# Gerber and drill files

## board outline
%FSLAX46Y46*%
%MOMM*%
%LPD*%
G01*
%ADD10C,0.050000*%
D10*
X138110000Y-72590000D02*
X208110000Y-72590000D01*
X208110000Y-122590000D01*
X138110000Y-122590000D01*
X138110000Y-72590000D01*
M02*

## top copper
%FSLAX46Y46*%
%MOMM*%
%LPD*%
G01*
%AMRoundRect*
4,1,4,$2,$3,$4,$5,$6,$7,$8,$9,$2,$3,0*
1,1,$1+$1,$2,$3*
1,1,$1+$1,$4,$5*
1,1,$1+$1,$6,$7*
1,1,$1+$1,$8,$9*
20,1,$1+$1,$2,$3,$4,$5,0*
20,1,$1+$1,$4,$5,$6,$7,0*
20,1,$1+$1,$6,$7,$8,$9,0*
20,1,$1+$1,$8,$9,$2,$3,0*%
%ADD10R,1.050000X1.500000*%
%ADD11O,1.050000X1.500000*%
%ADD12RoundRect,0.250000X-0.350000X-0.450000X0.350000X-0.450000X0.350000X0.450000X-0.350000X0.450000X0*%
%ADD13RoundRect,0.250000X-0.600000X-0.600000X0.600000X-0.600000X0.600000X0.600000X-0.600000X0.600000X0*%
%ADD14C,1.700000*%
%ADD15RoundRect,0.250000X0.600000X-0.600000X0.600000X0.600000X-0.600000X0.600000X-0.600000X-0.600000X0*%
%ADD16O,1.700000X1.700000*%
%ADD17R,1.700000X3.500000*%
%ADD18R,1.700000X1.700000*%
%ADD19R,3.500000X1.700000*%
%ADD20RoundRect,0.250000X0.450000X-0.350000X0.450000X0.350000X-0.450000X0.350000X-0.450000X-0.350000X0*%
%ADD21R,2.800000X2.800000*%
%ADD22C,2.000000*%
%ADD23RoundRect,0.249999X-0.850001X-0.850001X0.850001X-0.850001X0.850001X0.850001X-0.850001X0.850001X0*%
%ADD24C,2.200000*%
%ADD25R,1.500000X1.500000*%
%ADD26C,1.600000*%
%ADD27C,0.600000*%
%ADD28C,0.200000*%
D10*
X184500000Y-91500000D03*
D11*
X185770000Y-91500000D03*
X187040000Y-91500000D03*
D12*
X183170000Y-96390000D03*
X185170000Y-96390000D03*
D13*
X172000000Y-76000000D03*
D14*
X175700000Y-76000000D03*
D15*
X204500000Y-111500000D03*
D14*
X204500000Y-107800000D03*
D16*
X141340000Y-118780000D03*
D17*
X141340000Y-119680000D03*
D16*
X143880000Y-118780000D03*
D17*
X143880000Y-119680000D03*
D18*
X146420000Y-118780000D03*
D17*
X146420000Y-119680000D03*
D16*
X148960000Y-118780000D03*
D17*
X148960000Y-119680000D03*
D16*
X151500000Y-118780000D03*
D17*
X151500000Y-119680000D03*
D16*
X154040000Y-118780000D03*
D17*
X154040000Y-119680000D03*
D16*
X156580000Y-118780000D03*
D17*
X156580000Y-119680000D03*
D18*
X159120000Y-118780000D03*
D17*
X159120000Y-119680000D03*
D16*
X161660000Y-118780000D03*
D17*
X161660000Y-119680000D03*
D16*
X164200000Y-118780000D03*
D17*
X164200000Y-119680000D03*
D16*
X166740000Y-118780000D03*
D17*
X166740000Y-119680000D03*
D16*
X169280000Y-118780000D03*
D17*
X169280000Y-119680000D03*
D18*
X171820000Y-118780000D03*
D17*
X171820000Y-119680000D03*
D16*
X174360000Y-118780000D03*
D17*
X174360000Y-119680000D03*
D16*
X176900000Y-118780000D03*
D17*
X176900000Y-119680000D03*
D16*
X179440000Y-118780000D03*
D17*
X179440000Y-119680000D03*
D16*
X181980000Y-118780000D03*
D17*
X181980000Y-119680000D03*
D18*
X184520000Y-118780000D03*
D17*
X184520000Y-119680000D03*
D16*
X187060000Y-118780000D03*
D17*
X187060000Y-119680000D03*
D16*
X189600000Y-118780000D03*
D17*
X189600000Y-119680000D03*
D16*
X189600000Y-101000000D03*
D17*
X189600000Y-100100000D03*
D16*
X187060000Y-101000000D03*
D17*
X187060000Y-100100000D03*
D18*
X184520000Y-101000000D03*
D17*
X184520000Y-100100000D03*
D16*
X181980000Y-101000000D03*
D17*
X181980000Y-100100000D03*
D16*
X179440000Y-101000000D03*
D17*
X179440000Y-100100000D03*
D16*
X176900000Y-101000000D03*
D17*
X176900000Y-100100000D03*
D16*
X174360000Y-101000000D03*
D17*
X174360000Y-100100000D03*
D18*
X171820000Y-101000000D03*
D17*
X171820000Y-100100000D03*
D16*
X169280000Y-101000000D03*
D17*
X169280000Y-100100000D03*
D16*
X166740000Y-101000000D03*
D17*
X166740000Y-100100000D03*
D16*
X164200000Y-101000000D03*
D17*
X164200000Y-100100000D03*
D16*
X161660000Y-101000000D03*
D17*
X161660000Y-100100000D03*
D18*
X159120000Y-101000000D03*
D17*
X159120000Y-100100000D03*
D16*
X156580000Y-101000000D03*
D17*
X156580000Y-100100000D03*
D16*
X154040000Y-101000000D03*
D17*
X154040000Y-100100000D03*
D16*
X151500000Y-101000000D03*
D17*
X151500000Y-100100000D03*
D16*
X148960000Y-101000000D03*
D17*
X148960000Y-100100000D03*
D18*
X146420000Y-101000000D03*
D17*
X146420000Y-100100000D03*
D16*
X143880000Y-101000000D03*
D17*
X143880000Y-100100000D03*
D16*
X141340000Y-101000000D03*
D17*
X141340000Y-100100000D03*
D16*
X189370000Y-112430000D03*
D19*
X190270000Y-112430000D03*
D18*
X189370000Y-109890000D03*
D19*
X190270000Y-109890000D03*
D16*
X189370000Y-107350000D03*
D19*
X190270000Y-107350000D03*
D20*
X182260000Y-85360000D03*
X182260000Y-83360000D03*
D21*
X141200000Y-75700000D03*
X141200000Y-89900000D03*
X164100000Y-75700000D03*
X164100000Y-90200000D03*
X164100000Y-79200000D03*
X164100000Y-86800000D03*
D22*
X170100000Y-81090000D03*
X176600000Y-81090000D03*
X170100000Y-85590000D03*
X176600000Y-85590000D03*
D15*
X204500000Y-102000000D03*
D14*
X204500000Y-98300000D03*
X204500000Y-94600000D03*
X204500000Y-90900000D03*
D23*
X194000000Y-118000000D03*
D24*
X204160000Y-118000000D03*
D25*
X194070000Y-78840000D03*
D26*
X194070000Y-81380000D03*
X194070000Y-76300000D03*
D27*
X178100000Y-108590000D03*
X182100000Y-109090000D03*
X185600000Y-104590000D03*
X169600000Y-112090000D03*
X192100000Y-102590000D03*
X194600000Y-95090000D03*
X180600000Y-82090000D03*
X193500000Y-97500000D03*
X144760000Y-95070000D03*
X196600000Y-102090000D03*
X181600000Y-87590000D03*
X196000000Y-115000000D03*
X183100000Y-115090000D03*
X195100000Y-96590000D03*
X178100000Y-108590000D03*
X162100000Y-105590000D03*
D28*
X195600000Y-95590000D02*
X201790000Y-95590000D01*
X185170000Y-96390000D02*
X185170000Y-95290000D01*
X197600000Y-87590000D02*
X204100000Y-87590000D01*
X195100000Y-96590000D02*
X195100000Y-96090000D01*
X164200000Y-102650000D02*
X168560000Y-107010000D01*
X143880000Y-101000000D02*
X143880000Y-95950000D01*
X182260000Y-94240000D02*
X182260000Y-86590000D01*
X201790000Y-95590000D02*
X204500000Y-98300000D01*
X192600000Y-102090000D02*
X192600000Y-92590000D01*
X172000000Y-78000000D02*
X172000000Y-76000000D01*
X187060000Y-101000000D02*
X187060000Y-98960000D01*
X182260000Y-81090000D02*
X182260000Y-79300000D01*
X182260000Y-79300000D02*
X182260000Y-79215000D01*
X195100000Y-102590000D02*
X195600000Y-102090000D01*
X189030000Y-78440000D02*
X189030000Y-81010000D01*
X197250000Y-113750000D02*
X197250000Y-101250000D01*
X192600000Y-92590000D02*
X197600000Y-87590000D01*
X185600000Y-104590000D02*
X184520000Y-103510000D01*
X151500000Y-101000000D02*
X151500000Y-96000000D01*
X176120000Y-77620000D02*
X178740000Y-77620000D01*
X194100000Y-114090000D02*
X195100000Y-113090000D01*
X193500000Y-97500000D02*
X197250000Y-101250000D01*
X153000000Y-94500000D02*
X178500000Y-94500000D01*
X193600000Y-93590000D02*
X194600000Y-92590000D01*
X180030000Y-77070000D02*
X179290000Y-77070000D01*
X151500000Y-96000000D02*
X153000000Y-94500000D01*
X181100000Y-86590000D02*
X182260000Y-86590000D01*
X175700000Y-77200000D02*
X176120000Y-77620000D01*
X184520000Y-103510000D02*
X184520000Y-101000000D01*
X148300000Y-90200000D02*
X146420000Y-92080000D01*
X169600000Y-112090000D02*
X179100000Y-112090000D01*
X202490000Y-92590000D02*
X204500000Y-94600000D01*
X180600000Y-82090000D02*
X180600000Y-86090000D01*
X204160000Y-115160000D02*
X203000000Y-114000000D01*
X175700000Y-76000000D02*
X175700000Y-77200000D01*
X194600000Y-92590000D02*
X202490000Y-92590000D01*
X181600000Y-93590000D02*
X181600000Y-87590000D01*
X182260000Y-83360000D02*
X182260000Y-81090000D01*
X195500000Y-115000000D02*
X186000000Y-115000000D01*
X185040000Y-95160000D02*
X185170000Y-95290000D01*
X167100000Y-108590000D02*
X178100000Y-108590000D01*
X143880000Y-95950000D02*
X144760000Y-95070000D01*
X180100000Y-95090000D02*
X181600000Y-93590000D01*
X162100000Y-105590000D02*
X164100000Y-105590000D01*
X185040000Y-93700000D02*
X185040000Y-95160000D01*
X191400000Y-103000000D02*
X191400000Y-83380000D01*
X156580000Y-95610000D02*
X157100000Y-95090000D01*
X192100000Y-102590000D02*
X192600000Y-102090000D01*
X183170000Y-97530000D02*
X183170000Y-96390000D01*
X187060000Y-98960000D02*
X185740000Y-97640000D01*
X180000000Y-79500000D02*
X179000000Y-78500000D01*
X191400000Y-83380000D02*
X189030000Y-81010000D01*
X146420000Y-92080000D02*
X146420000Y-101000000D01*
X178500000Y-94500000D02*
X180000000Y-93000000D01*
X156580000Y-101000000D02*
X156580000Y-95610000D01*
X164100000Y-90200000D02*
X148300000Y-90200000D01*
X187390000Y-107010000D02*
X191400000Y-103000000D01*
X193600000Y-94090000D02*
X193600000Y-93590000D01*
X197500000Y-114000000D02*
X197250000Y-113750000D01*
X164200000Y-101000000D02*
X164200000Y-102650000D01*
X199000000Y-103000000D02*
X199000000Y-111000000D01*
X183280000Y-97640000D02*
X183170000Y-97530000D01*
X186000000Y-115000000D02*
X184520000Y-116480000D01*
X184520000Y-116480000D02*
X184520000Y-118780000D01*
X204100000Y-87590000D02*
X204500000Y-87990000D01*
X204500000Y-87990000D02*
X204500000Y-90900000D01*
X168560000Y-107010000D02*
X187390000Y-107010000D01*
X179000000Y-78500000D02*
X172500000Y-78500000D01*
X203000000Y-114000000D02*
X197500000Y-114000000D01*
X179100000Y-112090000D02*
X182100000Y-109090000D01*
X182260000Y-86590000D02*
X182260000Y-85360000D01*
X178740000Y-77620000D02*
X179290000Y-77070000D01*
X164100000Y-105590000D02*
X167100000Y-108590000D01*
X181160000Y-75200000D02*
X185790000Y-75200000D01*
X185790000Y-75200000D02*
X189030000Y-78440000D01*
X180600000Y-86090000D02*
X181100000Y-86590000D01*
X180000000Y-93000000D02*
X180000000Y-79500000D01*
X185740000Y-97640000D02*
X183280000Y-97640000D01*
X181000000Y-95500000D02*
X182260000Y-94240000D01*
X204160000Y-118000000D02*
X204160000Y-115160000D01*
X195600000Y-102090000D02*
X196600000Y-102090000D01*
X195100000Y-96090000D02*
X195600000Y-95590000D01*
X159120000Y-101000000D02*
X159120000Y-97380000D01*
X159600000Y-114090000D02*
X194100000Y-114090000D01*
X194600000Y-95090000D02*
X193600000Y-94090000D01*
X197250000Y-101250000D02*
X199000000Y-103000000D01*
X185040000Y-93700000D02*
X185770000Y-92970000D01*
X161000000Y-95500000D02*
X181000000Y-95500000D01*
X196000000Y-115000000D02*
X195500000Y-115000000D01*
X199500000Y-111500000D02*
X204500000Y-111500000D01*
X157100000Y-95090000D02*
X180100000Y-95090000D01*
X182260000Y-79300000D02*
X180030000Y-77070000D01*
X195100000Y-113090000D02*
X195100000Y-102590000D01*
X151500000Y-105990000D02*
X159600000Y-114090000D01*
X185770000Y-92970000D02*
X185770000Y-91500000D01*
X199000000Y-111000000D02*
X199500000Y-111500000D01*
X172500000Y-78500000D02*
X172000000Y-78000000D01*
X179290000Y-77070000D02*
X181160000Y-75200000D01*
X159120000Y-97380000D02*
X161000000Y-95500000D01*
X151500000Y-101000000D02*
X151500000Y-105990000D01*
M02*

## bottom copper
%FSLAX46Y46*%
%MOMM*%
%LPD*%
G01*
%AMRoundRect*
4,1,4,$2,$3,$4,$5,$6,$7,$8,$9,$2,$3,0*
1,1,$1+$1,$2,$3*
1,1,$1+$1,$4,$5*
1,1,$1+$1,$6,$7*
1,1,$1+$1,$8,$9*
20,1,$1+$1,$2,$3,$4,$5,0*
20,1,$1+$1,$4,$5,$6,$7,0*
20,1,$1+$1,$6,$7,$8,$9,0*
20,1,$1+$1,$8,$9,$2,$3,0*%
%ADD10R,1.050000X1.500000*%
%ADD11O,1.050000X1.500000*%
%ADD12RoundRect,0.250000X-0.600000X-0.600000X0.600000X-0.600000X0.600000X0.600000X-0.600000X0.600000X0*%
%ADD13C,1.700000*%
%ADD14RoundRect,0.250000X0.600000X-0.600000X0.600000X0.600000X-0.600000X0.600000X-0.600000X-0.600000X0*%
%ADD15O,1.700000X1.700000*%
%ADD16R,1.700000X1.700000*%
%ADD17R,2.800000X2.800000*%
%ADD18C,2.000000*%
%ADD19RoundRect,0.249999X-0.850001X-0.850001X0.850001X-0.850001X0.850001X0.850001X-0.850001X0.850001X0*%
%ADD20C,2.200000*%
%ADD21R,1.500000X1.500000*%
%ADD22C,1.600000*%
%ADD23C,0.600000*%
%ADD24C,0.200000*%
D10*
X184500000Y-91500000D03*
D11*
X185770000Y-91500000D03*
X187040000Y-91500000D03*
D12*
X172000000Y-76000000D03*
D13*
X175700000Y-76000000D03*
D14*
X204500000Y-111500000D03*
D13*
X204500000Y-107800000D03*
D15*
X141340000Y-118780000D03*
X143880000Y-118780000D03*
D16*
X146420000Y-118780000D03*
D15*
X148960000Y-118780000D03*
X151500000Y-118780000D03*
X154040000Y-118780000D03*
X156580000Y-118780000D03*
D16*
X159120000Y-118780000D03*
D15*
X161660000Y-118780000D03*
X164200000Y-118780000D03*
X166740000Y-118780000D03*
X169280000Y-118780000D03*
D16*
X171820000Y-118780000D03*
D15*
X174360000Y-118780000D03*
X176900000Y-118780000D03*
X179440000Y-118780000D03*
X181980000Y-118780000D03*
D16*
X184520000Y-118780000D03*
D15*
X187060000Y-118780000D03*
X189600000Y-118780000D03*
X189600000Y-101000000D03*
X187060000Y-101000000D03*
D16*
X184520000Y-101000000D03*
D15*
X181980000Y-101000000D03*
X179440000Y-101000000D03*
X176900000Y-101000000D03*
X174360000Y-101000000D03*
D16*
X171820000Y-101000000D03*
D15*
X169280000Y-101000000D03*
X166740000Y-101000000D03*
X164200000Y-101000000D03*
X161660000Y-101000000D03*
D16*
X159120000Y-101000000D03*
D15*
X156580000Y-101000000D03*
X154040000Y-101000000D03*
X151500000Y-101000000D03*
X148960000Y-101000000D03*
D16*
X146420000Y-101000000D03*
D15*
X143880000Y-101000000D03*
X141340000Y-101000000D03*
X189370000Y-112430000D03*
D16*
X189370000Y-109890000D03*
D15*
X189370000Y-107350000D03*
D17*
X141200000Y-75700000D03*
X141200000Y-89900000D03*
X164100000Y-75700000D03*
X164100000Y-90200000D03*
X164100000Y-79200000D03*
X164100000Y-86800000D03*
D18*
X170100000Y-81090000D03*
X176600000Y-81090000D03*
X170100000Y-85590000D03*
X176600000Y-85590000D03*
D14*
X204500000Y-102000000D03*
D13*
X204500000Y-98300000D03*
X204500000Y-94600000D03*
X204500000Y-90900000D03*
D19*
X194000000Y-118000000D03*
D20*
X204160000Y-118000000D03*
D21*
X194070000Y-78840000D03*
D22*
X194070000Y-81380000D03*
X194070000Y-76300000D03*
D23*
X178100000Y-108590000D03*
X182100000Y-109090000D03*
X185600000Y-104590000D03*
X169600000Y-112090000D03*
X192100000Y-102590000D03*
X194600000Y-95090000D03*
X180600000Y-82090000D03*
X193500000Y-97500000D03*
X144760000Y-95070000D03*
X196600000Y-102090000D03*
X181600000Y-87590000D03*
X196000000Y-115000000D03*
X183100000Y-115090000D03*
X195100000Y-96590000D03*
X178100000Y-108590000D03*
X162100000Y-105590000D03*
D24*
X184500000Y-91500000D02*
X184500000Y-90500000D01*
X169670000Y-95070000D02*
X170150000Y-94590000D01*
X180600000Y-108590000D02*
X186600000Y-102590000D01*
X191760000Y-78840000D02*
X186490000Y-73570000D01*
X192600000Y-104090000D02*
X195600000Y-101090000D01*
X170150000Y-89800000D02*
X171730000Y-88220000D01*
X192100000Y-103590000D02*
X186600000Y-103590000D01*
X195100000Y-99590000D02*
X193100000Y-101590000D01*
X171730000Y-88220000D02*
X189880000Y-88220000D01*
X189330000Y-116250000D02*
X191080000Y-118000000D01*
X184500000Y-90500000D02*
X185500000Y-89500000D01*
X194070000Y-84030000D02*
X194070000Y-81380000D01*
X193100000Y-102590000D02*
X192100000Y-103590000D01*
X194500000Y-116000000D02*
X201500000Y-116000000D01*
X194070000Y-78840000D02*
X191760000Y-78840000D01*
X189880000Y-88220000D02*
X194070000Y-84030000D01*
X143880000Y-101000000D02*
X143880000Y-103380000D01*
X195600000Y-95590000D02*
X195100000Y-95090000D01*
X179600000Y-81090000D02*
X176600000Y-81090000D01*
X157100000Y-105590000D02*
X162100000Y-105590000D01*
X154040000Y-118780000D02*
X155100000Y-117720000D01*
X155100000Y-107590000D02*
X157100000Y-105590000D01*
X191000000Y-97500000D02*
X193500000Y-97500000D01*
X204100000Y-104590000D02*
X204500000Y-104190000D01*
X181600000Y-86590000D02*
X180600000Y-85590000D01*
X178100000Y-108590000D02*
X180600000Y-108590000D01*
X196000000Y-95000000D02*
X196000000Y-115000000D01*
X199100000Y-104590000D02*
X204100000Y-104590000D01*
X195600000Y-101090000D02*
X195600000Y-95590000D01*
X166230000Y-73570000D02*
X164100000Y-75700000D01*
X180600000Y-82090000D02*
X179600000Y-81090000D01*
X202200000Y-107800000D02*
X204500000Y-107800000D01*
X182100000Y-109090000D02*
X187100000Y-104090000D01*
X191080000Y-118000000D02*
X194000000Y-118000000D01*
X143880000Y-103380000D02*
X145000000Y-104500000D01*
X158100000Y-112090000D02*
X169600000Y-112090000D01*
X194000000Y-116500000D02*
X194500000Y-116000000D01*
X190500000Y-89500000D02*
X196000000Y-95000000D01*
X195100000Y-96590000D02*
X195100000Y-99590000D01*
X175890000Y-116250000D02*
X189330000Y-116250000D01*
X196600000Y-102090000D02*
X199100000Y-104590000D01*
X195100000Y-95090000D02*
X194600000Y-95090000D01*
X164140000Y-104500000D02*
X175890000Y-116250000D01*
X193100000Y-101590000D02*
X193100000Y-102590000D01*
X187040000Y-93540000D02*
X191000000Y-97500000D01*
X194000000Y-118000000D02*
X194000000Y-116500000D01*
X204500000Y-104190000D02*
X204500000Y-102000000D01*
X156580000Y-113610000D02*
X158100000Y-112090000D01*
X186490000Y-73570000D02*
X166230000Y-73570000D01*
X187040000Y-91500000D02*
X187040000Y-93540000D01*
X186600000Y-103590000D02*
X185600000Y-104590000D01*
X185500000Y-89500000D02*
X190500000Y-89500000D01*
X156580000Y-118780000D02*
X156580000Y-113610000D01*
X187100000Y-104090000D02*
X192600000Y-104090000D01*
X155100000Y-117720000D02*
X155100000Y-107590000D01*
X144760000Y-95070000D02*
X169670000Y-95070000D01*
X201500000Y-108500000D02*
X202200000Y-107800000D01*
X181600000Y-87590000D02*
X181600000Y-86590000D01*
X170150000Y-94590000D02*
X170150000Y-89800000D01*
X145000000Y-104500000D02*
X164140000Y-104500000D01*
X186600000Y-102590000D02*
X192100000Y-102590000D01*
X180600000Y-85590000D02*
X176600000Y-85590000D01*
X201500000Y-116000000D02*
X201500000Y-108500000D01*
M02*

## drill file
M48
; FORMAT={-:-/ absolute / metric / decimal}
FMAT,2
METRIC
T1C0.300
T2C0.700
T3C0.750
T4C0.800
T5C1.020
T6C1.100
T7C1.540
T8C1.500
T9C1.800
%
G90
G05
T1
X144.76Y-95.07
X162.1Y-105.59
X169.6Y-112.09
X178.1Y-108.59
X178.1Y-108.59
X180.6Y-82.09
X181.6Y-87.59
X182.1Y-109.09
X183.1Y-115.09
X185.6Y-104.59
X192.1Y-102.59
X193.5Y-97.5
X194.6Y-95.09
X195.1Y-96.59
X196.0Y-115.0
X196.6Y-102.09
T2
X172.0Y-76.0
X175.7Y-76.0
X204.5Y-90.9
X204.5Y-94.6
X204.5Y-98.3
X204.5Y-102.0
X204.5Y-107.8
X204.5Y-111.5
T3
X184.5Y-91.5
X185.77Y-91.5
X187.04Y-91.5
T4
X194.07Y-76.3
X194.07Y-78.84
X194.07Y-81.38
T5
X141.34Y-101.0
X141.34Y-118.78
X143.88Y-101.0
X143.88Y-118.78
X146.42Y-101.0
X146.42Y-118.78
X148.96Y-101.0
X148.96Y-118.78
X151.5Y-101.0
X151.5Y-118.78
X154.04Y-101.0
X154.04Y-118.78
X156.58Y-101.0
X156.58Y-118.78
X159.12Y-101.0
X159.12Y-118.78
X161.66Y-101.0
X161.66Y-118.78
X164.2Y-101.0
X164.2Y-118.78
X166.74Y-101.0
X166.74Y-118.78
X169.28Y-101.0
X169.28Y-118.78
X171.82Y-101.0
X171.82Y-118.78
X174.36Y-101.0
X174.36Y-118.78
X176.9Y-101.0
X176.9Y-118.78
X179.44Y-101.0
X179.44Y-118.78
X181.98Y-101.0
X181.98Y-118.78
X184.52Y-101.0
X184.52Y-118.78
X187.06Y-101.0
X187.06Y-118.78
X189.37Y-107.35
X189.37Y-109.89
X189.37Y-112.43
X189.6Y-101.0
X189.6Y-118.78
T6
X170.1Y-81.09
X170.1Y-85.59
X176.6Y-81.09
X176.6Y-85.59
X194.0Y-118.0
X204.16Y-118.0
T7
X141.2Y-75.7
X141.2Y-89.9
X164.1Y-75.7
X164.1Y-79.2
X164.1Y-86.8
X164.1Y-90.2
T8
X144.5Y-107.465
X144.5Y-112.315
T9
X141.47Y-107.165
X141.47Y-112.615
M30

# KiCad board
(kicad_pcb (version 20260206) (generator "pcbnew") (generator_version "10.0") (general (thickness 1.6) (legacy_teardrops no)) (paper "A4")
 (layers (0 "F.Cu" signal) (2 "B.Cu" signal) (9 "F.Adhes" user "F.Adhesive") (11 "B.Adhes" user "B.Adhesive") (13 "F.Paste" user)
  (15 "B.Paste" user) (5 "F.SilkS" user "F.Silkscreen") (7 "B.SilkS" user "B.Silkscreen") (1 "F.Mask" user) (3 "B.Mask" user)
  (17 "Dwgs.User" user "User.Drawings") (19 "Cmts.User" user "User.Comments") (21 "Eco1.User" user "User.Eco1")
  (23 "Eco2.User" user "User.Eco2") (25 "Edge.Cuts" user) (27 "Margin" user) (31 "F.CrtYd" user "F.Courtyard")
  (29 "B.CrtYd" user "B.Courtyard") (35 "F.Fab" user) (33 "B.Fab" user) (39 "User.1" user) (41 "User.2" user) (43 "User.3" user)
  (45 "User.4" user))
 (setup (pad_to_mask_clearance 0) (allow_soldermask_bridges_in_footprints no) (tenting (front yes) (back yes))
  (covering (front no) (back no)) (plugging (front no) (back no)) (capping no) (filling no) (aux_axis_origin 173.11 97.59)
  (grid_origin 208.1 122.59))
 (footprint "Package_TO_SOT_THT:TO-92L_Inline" (layer "F.Cu") (at 184.5 91.5)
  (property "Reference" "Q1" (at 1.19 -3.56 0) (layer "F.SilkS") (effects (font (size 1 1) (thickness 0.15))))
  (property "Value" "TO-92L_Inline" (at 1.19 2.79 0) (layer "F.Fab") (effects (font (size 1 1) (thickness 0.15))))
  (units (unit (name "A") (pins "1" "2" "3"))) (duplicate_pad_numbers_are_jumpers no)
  (pad "1" thru_hole rect (at 0 0) (size 1.05 1.5) (drill 0.75) (layers "*.Cu" "*.Mask") (remove_unused_layers no))
  (pad "2" thru_hole oval (at 1.27 0) (size 1.05 1.5) (drill 0.75) (layers "*.Cu" "*.Mask") (remove_unused_layers no))
  (pad "3" thru_hole oval (at 2.54 0) (size 1.05 1.5) (drill 0.75) (layers "*.Cu" "*.Mask") (remove_unused_layers no)))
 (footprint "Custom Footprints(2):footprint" (layer "F.Cu") (at 202 78.55)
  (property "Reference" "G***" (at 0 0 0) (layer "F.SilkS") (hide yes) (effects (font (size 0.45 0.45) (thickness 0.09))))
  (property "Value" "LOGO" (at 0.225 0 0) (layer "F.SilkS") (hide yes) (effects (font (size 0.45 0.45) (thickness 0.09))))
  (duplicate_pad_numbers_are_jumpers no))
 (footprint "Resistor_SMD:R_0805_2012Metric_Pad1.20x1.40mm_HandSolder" (layer "F.Cu") (at 184.17 96.39)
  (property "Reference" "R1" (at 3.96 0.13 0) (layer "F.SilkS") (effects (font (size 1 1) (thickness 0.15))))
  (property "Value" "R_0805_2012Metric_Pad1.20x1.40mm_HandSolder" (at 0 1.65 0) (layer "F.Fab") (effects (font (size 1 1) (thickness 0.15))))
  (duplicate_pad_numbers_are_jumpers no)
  (pad "1" smd roundrect (at -1 0) (size 1.2 1.4) (layers "F.Cu" "F.Mask" "F.Paste") (roundrect_rratio 0.208333))
  (pad "2" smd roundrect (at 1 0) (size 1.2 1.4) (layers "F.Cu" "F.Mask" "F.Paste") (roundrect_rratio 0.208333)))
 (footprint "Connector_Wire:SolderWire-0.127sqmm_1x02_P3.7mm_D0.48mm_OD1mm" (layer "F.Cu") (at 172 76)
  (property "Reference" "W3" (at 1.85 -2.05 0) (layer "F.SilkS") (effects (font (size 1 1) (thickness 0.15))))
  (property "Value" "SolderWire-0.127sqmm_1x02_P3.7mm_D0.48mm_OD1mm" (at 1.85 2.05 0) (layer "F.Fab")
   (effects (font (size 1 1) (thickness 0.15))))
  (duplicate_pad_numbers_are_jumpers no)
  (pad "1" thru_hole roundrect (at 0 0) (size 1.7 1.7) (drill 0.7) (layers "*.Cu" "*.Mask") (remove_unused_layers no)
   (roundrect_rratio 0.147059))
  (pad "2" thru_hole circle (at 3.7 0) (size 1.7 1.7) (drill 0.7) (layers "*.Cu" "*.Mask") (remove_unused_layers no)))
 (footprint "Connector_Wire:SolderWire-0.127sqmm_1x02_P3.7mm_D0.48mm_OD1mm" (layer "F.Cu") (at 204.5 111.5 90)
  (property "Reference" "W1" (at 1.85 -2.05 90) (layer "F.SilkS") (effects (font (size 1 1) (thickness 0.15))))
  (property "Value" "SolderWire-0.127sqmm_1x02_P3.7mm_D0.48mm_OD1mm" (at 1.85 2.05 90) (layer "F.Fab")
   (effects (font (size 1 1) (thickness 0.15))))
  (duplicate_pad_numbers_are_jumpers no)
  (pad "1" thru_hole roundrect (at 0 0 90) (size 1.7 1.7) (drill 0.7) (layers "*.Cu" "*.Mask") (remove_unused_layers no)
   (roundrect_rratio 0.147059))
  (pad "2" thru_hole circle (at 3.7 0 90) (size 1.7 1.7) (drill 0.7) (layers "*.Cu" "*.Mask") (remove_unused_layers no)))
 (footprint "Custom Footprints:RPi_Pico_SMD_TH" (layer "F.Cu") (at 165.47 109.89 90)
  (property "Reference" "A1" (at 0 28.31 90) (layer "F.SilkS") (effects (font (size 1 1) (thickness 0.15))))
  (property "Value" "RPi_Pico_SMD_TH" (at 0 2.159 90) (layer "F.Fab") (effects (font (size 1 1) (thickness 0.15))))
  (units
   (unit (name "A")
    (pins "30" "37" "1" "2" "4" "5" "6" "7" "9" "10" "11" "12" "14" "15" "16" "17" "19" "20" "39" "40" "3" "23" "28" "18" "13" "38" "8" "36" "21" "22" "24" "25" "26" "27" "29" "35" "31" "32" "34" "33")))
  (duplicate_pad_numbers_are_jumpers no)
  (pad "" np_thru_hole oval (at -2.725 -24 90) (size 1.8 1.8) (drill 1.8) (layers "*.Cu" "*.Mask"))
  (pad "" np_thru_hole oval (at -2.425 -20.97 90) (size 1.5 1.5) (drill 1.5) (layers "*.Cu" "*.Mask"))
  (pad "" np_thru_hole oval (at 2.425 -20.97 90) (size 1.5 1.5) (drill 1.5) (layers "*.Cu" "*.Mask"))
  (pad "" np_thru_hole oval (at 2.725 -24 90) (size 1.8 1.8) (drill 1.8) (layers "*.Cu" "*.Mask"))
  (pad "1" thru_hole oval (at -8.89 -24.13 90) (size 1.7 1.7) (drill 1.02) (layers "*.Cu" "*.Mask") (remove_unused_layers no))
  (pad "1" smd rect (at -8.89 -24.13 90) (size 3.5 1.7) (drill (offset -0.9 0)) (layers "F.Cu" "F.Mask"))
  (pad "2" thru_hole oval (at -8.89 -21.59 90) (size 1.7 1.7) (drill 1.02) (layers "*.Cu" "*.Mask") (remove_unused_layers no))
  (pad "2" smd rect (at -8.89 -21.59 90) (size 3.5 1.7) (drill (offset -0.9 0)) (layers "F.Cu" "F.Mask"))
  (pad "3" thru_hole rect (at -8.89 -19.05 90) (size 1.7 1.7) (drill 1.02) (layers "*.Cu" "*.Mask") (remove_unused_layers no))
  (pad "3" smd rect (at -8.89 -19.05 90) (size 3.5 1.7) (drill (offset -0.9 0)) (layers "F.Cu" "F.Mask"))
  (pad "4" thru_hole oval (at -8.89 -16.51 90) (size 1.7 1.7) (drill 1.02) (layers "*.Cu" "*.Mask") (remove_unused_layers no))
  (pad "4" smd rect (at -8.89 -16.51 90) (size 3.5 1.7) (drill (offset -0.9 0)) (layers "F.Cu" "F.Mask"))
  (pad "5" thru_hole oval (at -8.89 -13.97 90) (size 1.7 1.7) (drill 1.02) (layers "*.Cu" "*.Mask") (remove_unused_layers no))
  (pad "5" smd rect (at -8.89 -13.97 90) (size 3.5 1.7) (drill (offset -0.9 0)) (layers "F.Cu" "F.Mask"))
  (pad "6" thru_hole oval (at -8.89 -11.43 90) (size 1.7 1.7) (drill 1.02) (layers "*.Cu" "*.Mask") (remove_unused_layers no))
  (pad "6" smd rect (at -8.89 -11.43 90) (size 3.5 1.7) (drill (offset -0.9 0)) (layers "F.Cu" "F.Mask"))
  (pad "7" thru_hole oval (at -8.89 -8.89 90) (size 1.7 1.7) (drill 1.02) (layers "*.Cu" "*.Mask") (remove_unused_layers no))
  (pad "7" smd rect (at -8.89 -8.89 90) (size 3.5 1.7) (drill (offset -0.9 0)) (layers "F.Cu" "F.Mask"))
  (pad "8" thru_hole rect (at -8.89 -6.35 90) (size 1.7 1.7) (drill 1.02) (layers "*.Cu" "*.Mask") (remove_unused_layers no))
  (pad "8" smd rect (at -8.89 -6.35 90) (size 3.5 1.7) (drill (offset -0.9 0)) (layers "F.Cu" "F.Mask"))
  (pad "9" thru_hole oval (at -8.89 -3.81 90) (size 1.7 1.7) (drill 1.02) (layers "*.Cu" "*.Mask") (remove_unused_layers no))
  (pad "9" smd rect (at -8.89 -3.81 90) (size 3.5 1.7) (drill (offset -0.9 0)) (layers "F.Cu" "F.Mask"))
  (pad "10" thru_hole oval (at -8.89 -1.27 90) (size 1.7 1.7) (drill 1.02) (layers "*.Cu" "*.Mask") (remove_unused_layers no))
  (pad "10" smd rect (at -8.89 -1.27 90) (size 3.5 1.7) (drill (offset -0.9 0)) (layers "F.Cu" "F.Mask"))
  (pad "11" thru_hole oval (at -8.89 1.27 90) (size 1.7 1.7) (drill 1.02) (layers "*.Cu" "*.Mask") (remove_unused_layers no))
  (pad "11" smd rect (at -8.89 1.27 90) (size 3.5 1.7) (drill (offset -0.9 0)) (layers "F.Cu" "F.Mask"))
  (pad "12" thru_hole oval (at -8.89 3.81 90) (size 1.7 1.7) (drill 1.02) (layers "*.Cu" "*.Mask") (remove_unused_layers no))
  (pad "12" smd rect (at -8.89 3.81 90) (size 3.5 1.7) (drill (offset -0.9 0)) (layers "F.Cu" "F.Mask"))
  (pad "13" thru_hole rect (at -8.89 6.35 90) (size 1.7 1.7) (drill 1.02) (layers "*.Cu" "*.Mask") (remove_unused_layers no))
  (pad "13" smd rect (at -8.89 6.35 90) (size 3.5 1.7) (drill (offset -0.9 0)) (layers "F.Cu" "F.Mask"))
  (pad "14" thru_hole oval (at -8.89 8.89 90) (size 1.7 1.7) (drill 1.02) (layers "*.Cu" "*.Mask") (remove_unused_layers no))
  (pad "14" smd rect (at -8.89 8.89 90) (size 3.5 1.7) (drill (offset -0.9 0)) (layers "F.Cu" "F.Mask"))
  (pad "15" thru_hole oval (at -8.89 11.43 90) (size 1.7 1.7) (drill 1.02) (layers "*.Cu" "*.Mask") (remove_unused_layers no))
  (pad "15" smd rect (at -8.89 11.43 90) (size 3.5 1.7) (drill (offset -0.9 0)) (layers "F.Cu" "F.Mask"))
  (pad "16" thru_hole oval (at -8.89 13.97 90) (size 1.7 1.7) (drill 1.02) (layers "*.Cu" "*.Mask") (remove_unused_layers no))
  (pad "16" smd rect (at -8.89 13.97 90) (size 3.5 1.7) (drill (offset -0.9 0)) (layers "F.Cu" "F.Mask"))
  (pad "17" thru_hole oval (at -8.89 16.51 90) (size 1.7 1.7) (drill 1.02) (layers "*.Cu" "*.Mask") (remove_unused_layers no))
  (pad "17" smd rect (at -8.89 16.51 90) (size 3.5 1.7) (drill (offset -0.9 0)) (layers "F.Cu" "F.Mask"))
  (pad "18" thru_hole rect (at -8.89 19.05 90) (size 1.7 1.7) (drill 1.02) (layers "*.Cu" "*.Mask") (remove_unused_layers no))
  (pad "18" smd rect (at -8.89 19.05 90) (size 3.5 1.7) (drill (offset -0.9 0)) (layers "F.Cu" "F.Mask"))
  (pad "19" thru_hole oval (at -8.89 21.59 90) (size 1.7 1.7) (drill 1.02) (layers "*.Cu" "*.Mask") (remove_unused_layers no))
  (pad "19" smd rect (at -8.89 21.59 90) (size 3.5 1.7) (drill (offset -0.9 0)) (layers "F.Cu" "F.Mask"))
  (pad "20" thru_hole oval (at -8.89 24.13 90) (size 1.7 1.7) (drill 1.02) (layers "*.Cu" "*.Mask") (remove_unused_layers no))
  (pad "20" smd rect (at -8.89 24.13 90) (size 3.5 1.7) (drill (offset -0.9 0)) (layers "F.Cu" "F.Mask"))
  (pad "21" thru_hole oval (at 8.89 24.13 90) (size 1.7 1.7) (drill 1.02) (layers "*.Cu" "*.Mask") (remove_unused_layers no))
  (pad "21" smd rect (at 8.89 24.13 90) (size 3.5 1.7) (drill (offset 0.9 0)) (layers "F.Cu" "F.Mask"))
  (pad "22" thru_hole oval (at 8.89 21.59 90) (size 1.7 1.7) (drill 1.02) (layers "*.Cu" "*.Mask") (remove_unused_layers no))
  (pad "22" smd rect (at 8.89 21.59 90) (size 3.5 1.7) (drill (offset 0.9 0)) (layers "F.Cu" "F.Mask"))
  (pad "23" thru_hole rect (at 8.89 19.05 90) (size 1.7 1.7) (drill 1.02) (layers "*.Cu" "*.Mask") (remove_unused_layers no))
  (pad "23" smd rect (at 8.89 19.05 90) (size 3.5 1.7) (drill (offset 0.9 0)) (layers "F.Cu" "F.Mask"))
  (pad "24" thru_hole oval (at 8.89 16.51 90) (size 1.7 1.7) (drill 1.02) (layers "*.Cu" "*.Mask") (remove_unused_layers no))
  (pad "24" smd rect (at 8.89 16.51 90) (size 3.5 1.7) (drill (offset 0.9 0)) (layers "F.Cu" "F.Mask"))
  (pad "25" thru_hole oval (at 8.89 13.97 90) (size 1.7 1.7) (drill 1.02) (layers "*.Cu" "*.Mask") (remove_unused_layers no))
  (pad "25" smd rect (at 8.89 13.97 90) (size 3.5 1.7) (drill (offset 0.9 0)) (layers "F.Cu" "F.Mask"))
  (pad "26" thru_hole oval (at 8.89 11.43 90) (size 1.7 1.7) (drill 1.02) (layers "*.Cu" "*.Mask") (remove_unused_layers no))
  (pad "26" smd rect (at 8.89 11.43 90) (size 3.5 1.7) (drill (offset 0.9 0)) (layers "F.Cu" "F.Mask"))
  (pad "27" thru_hole oval (at 8.89 8.89 90) (size 1.7 1.7) (drill 1.02) (layers "*.Cu" "*.Mask") (remove_unused_layers no))
  (pad "27" smd rect (at 8.89 8.89 90) (size 3.5 1.7) (drill (offset 0.9 0)) (layers "F.Cu" "F.Mask"))
  (pad "28" thru_hole rect (at 8.89 6.35 90) (size 1.7 1.7) (drill 1.02) (layers "*.Cu" "*.Mask") (remove_unused_layers no))
  (pad "28" smd rect (at 8.89 6.35 90) (size 3.5 1.7) (drill (offset 0.9 0)) (layers "F.Cu" "F.Mask"))
  (pad "29" thru_hole oval (at 8.89 3.81 90) (size 1.7 1.7) (drill 1.02) (layers "*.Cu" "*.Mask") (remove_unused_layers no))
  (pad "29" smd rect (at 8.89 3.81 90) (size 3.5 1.7) (drill (offset 0.9 0)) (layers "F.Cu" "F.Mask"))
  (pad "30" thru_hole oval (at 8.89 1.27 90) (size 1.7 1.7) (drill 1.02) (layers "*.Cu" "*.Mask") (remove_unused_layers no))
  (pad "30" smd rect (at 8.89 1.27 90) (size 3.5 1.7) (drill (offset 0.9 0)) (layers "F.Cu" "F.Mask"))
  (pad "31" thru_hole oval (at 8.89 -1.27 90) (size 1.7 1.7) (drill 1.02) (layers "*.Cu" "*.Mask") (remove_unused_layers no))
  (pad "31" smd rect (at 8.89 -1.27 90) (size 3.5 1.7) (drill (offset 0.9 0)) (layers "F.Cu" "F.Mask"))
  (pad "32" thru_hole oval (at 8.89 -3.81 90) (size 1.7 1.7) (drill 1.02) (layers "*.Cu" "*.Mask") (remove_unused_layers no))
  (pad "32" smd rect (at 8.89 -3.81 90) (size 3.5 1.7) (drill (offset 0.9 0)) (layers "F.Cu" "F.Mask"))
  (pad "33" thru_hole rect (at 8.89 -6.35 90) (size 1.7 1.7) (drill 1.02) (layers "*.Cu" "*.Mask") (remove_unused_layers no))
  (pad "33" smd rect (at 8.89 -6.35 90) (size 3.5 1.7) (drill (offset 0.9 0)) (layers "F.Cu" "F.Mask"))
  (pad "34" thru_hole oval (at 8.89 -8.89 90) (size 1.7 1.7) (drill 1.02) (layers "*.Cu" "*.Mask") (remove_unused_layers no))
  (pad "34" smd rect (at 8.89 -8.89 90) (size 3.5 1.7) (drill (offset 0.9 0)) (layers "F.Cu" "F.Mask"))
  (pad "35" thru_hole oval (at 8.89 -11.43 90) (size 1.7 1.7) (drill 1.02) (layers "*.Cu" "*.Mask") (remove_unused_layers no))
  (pad "35" smd rect (at 8.89 -11.43 90) (size 3.5 1.7) (drill (offset 0.9 0)) (layers "F.Cu" "F.Mask"))
  (pad "36" thru_hole oval (at 8.89 -13.97 90) (size 1.7 1.7) (drill 1.02) (layers "*.Cu" "*.Mask") (remove_unused_layers no))
  (pad "36" smd rect (at 8.89 -13.97 90) (size 3.5 1.7) (drill (offset 0.9 0)) (layers "F.Cu" "F.Mask"))
  (pad "37" thru_hole oval (at 8.89 -16.51 90) (size 1.7 1.7) (drill 1.02) (layers "*.Cu" "*.Mask") (remove_unused_layers no))
  (pad "37" smd rect (at 8.89 -16.51 90) (size 3.5 1.7) (drill (offset 0.9 0)) (layers "F.Cu" "F.Mask"))
  (pad "38" thru_hole rect (at 8.89 -19.05 90) (size 1.7 1.7) (drill 1.02) (layers "*.Cu" "*.Mask") (remove_unused_layers no))
  (pad "38" smd rect (at 8.89 -19.05 90) (size 3.5 1.7) (drill (offset 0.9 0)) (layers "F.Cu" "F.Mask"))
  (pad "39" thru_hole oval (at 8.89 -21.59 90) (size 1.7 1.7) (drill 1.02) (layers "*.Cu" "*.Mask") (remove_unused_layers no))
  (pad "39" smd rect (at 8.89 -21.59 90) (size 3.5 1.7) (drill (offset 0.9 0)) (layers "F.Cu" "F.Mask"))
  (pad "40" thru_hole oval (at 8.89 -24.13 90) (size 1.7 1.7) (drill 1.02) (layers "*.Cu" "*.Mask") (remove_unused_layers no))
  (pad "40" smd rect (at 8.89 -24.13 90) (size 3.5 1.7) (drill (offset 0.9 0)) (layers "F.Cu" "F.Mask"))
  (pad "41" thru_hole oval (at -2.54 23.9 90) (size 1.7 1.7) (drill 1.02) (layers "*.Cu" "*.Mask") (remove_unused_layers no))
  (pad "41" smd rect (at -2.54 23.9 180) (size 3.5 1.7) (drill (offset -0.9 0)) (layers "F.Cu" "F.Mask"))
  (pad "42" thru_hole rect (at 0 23.9 90) (size 1.7 1.7) (drill 1.02) (layers "*.Cu" "*.Mask") (remove_unused_layers no))
  (pad "42" smd rect (at 0 23.9 180) (size 3.5 1.7) (drill (offset -0.9 0)) (layers "F.Cu" "F.Mask"))
  (pad "43" thru_hole oval (at 2.54 23.9 90) (size 1.7 1.7) (drill 1.02) (layers "*.Cu" "*.Mask") (remove_unused_layers no))
  (pad "43" smd rect (at 2.54 23.9 180) (size 3.5 1.7) (drill (offset -0.9 0)) (layers "F.Cu" "F.Mask")))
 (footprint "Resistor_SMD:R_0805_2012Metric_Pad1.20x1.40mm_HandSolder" (layer "F.Cu") (at 182.26 84.36 90)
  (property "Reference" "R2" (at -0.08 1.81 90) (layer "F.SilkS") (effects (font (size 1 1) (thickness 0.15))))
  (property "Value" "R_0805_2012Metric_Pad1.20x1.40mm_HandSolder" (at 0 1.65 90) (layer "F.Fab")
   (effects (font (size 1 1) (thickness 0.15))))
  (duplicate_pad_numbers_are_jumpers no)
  (pad "1" smd roundrect (at -1 0 90) (size 1.2 1.4) (layers "F.Cu" "F.Mask" "F.Paste") (roundrect_rratio 0.208333))
  (pad "2" smd roundrect (at 1 0 90) (size 1.2 1.4) (layers "F.Cu" "F.Mask" "F.Paste") (roundrect_rratio 0.208333)))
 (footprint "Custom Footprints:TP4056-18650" (layer "F.Cu") (at 139.5 74)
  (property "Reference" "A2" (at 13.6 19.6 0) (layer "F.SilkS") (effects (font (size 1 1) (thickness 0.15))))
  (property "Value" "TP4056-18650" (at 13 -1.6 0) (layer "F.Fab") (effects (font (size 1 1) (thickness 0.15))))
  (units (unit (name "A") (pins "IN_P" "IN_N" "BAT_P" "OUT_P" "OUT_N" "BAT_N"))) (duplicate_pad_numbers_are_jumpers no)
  (pad "1" thru_hole rect (at 1.7 1.7) (size 2.8 2.8) (drill 1.54) (layers "*.Cu" "*.Mask") (remove_unused_layers no))
  (pad "2" thru_hole rect (at 1.7 15.9) (size 2.8 2.8) (drill 1.54) (layers "*.Cu" "*.Mask") (remove_unused_layers no))
  (pad "3" thru_hole rect (at 24.6 1.7) (size 2.8 2.8) (drill 1.54) (layers "*.Cu" "*.Mask") (remove_unused_layers no))
  (pad "4" thru_hole rect (at 24.6 16.2) (size 2.8 2.8) (drill 1.54) (layers "*.Cu" "*.Mask") (remove_unused_layers no))
  (pad "5" thru_hole rect (at 24.6 5.2) (size 2.8 2.8) (drill 1.54) (layers "*.Cu" "*.Mask") (remove_unused_layers no))
  (pad "6" thru_hole rect (at 24.6 12.8) (size 2.8 2.8) (drill 1.54) (layers "*.Cu" "*.Mask") (remove_unused_layers no)))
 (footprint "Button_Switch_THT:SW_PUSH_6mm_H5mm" (layer "F.Cu") (at 170.1 81.09)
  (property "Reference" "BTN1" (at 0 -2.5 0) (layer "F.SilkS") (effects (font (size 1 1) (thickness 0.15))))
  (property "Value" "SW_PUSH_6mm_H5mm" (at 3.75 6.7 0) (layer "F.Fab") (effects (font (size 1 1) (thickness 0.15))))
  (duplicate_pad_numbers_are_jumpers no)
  (pad "1" thru_hole circle (at 0 0 90) (size 2 2) (drill 1.1) (layers "*.Cu" "*.Mask") (remove_unused_layers no))
  (pad "1" thru_hole circle (at 6.5 0 90) (size 2 2) (drill 1.1) (layers "*.Cu" "*.Mask") (remove_unused_layers no))
  (pad "2" thru_hole circle (at 0 4.5 90) (size 2 2) (drill 1.1) (layers "*.Cu" "*.Mask") (remove_unused_layers no))
  (pad "2" thru_hole circle (at 6.5 4.5 90) (size 2 2) (drill 1.1) (layers "*.Cu" "*.Mask") (remove_unused_layers no)))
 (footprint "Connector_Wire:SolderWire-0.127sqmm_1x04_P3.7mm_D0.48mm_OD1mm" (layer "F.Cu") (at 204.5 102 90)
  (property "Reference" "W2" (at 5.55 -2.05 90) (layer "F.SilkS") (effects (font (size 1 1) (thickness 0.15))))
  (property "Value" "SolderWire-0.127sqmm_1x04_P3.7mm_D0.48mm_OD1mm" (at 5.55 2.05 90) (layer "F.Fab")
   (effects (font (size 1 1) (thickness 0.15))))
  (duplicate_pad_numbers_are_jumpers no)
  (pad "1" thru_hole roundrect (at 0 0 90) (size 1.7 1.7) (drill 0.7) (layers "*.Cu" "*.Mask") (remove_unused_layers no)
   (roundrect_rratio 0.147059))
  (pad "2" thru_hole circle (at 3.7 0 90) (size 1.7 1.7) (drill 0.7) (layers "*.Cu" "*.Mask") (remove_unused_layers no))
  (pad "3" thru_hole circle (at 7.4 0 90) (size 1.7 1.7) (drill 0.7) (layers "*.Cu" "*.Mask") (remove_unused_layers no))
  (pad "4" thru_hole circle (at 11.1 0 90) (size 1.7 1.7) (drill 0.7) (layers "*.Cu" "*.Mask") (remove_unused_layers no)))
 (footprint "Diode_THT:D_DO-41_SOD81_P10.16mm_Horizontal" (layer "F.Cu") (at 194 118)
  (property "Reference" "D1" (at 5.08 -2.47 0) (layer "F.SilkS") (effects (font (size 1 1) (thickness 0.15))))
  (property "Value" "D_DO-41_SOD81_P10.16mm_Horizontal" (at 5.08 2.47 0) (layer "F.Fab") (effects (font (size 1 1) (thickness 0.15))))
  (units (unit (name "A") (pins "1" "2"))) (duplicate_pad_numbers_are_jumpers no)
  (pad "1" thru_hole roundrect (at 0 0) (size 2.2 2.2) (drill 1.1) (layers "*.Cu" "*.Mask") (remove_unused_layers no)
   (roundrect_rratio 0.113636))
  (pad "2" thru_hole circle (at 10.16 0) (size 2.2 2.2) (drill 1.1) (layers "*.Cu" "*.Mask") (remove_unused_layers no)))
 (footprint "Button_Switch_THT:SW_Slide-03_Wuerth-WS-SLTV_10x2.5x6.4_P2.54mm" (layer "F.Cu") (at 194.07 78.84 90)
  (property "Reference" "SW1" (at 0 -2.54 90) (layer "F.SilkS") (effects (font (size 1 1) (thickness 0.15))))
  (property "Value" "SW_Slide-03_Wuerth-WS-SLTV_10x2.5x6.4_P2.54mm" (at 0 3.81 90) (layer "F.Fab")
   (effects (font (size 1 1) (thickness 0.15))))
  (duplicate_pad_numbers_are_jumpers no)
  (pad "1" thru_hole rect (at 0 0 90) (size 1.5 1.5) (drill 0.8) (layers "*.Cu" "*.Mask") (remove_unused_layers no))
  (pad "2" thru_hole circle (at -2.54 0 90) (size 1.6 1.6) (drill 0.8) (layers "*.Cu" "*.Mask") (remove_unused_layers no))
  (pad "3" thru_hole circle (at 2.54 0 90) (size 1.6 1.6) (drill 0.8) (layers "*.Cu" "*.Mask") (remove_unused_layers no)))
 (gr_rect (start 138.11 72.59) (end 208.11 122.59) (stroke (width 0.05) (type default)) (fill no) (layer "Edge.Cuts"))
 (segment (start 195.6 95.59) (end 201.79 95.59) (width 0.2) (layer "F.Cu") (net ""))
 (segment (start 185.17 96.39) (end 185.17 95.29) (width 0.2) (layer "F.Cu") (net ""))
 (segment (start 197.6 87.59) (end 204.1 87.59) (width 0.2) (layer "F.Cu") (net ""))
 (segment (start 195.1 96.59) (end 195.1 96.09) (width 0.2) (layer "F.Cu") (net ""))
 (segment (start 164.2 102.65) (end 168.56 107.01) (width 0.2) (layer "F.Cu") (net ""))
 (segment (start 143.88 101) (end 143.88 95.95) (width 0.2) (layer "F.Cu") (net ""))
 (segment (start 182.26 94.24) (end 182.26 86.59) (width 0.2) (layer "F.Cu") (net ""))
 (segment (start 201.79 95.59) (end 204.5 98.3) (width 0.2) (layer "F.Cu") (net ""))
 (segment (start 192.6 102.09) (end 192.6 92.59) (width 0.2) (layer "F.Cu") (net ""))
 (segment (start 172 78) (end 172 76) (width 0.2) (layer "F.Cu") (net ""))
 (segment (start 187.06 101) (end 187.06 98.96) (width 0.2) (layer "F.Cu") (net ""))
 (segment (start 182.26 81.09) (end 182.26 79.3) (width 0.2) (layer "F.Cu") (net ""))
 (segment (start 182.26 79.3) (end 182.26 79.215) (width 0.2) (layer "F.Cu") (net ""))
 (segment (start 195.1 102.59) (end 195.6 102.09) (width 0.2) (layer "F.Cu") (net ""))
 (segment (start 189.03 78.44) (end 189.03 81.01) (width 0.2) (layer "F.Cu") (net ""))
 (segment (start 197.25 113.75) (end 197.25 101.25) (width 0.2) (layer "F.Cu") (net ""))
 (segment (start 192.6 92.59) (end 197.6 87.59) (width 0.2) (layer "F.Cu") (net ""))
 (segment (start 185.6 104.59) (end 184.52 103.51) (width 0.2) (layer "F.Cu") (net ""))
 (segment (start 151.5 101) (end 151.5 96) (width 0.2) (layer "F.Cu") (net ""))
 (segment (start 176.12 77.62) (end 178.74 77.62) (width 0.2) (layer "F.Cu") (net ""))
 (segment (start 194.1 114.09) (end 195.1 113.09) (width 0.2) (layer "F.Cu") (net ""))
 (segment (start 193.5 97.5) (end 197.25 101.25) (width 0.2) (layer "F.Cu") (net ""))
 (segment (start 153 94.5) (end 178.5 94.5) (width 0.2) (layer "F.Cu") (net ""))
 (segment (start 193.6 93.59) (end 194.6 92.59) (width 0.2) (layer "F.Cu") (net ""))
 (segment (start 180.03 77.07) (end 179.29 77.07) (width 0.2) (layer "F.Cu") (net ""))
 (segment (start 151.5 96) (end 153 94.5) (width 0.2) (layer "F.Cu") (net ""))
 (segment (start 181.1 86.59) (end 182.26 86.59) (width 0.2) (layer "F.Cu") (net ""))
 (segment (start 175.7 77.2) (end 176.12 77.62) (width 0.2) (layer "F.Cu") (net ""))
 (segment (start 184.52 103.51) (end 184.52 101) (width 0.2) (layer "F.Cu") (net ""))
 (segment (start 148.3 90.2) (end 146.42 92.08) (width 0.2) (layer "F.Cu") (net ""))
 (segment (start 169.6 112.09) (end 179.1 112.09) (width 0.2) (layer "F.Cu") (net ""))
 (segment (start 202.49 92.59) (end 204.5 94.6) (width 0.2) (layer "F.Cu") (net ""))
 (segment (start 180.6 82.09) (end 180.6 86.09) (width 0.2) (layer "F.Cu") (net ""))
 (segment (start 204.16 115.16) (end 203 114) (width 0.2) (layer "F.Cu") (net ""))
 (segment (start 175.7 76) (end 175.7 77.2) (width 0.2) (layer "F.Cu") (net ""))
 (segment (start 194.6 92.59) (end 202.49 92.59) (width 0.2) (layer "F.Cu") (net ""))
 (segment (start 181.6 93.59) (end 181.6 87.59) (width 0.2) (layer "F.Cu") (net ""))
 (segment (start 182.26 83.36) (end 182.26 81.09) (width 0.2) (layer "F.Cu") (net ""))
 (segment (start 195.5 115) (end 186 115) (width 0.2) (layer "F.Cu") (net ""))
 (segment (start 185.04 95.16) (end 185.17 95.29) (width 0.2) (layer "F.Cu") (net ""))
 (segment (start 167.1 108.59) (end 178.1 108.59) (width 0.2) (layer "F.Cu") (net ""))
 (segment (start 143.88 95.95) (end 144.76 95.07) (width 0.2) (layer "F.Cu") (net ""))
 (segment (start 180.1 95.09) (end 181.6 93.59) (width 0.2) (layer "F.Cu") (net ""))
 (segment (start 162.1 105.59) (end 164.1 105.59) (width 0.2) (layer "F.Cu") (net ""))
 (segment (start 185.04 93.7) (end 185.04 95.16) (width 0.2) (layer "F.Cu") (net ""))
 (segment (start 191.4 103) (end 191.4 83.38) (width 0.2) (layer "F.Cu") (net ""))
 (segment (start 156.58 95.61) (end 157.1 95.09) (width 0.2) (layer "F.Cu") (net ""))
 (segment (start 192.1 102.59) (end 192.6 102.09) (width 0.2) (layer "F.Cu") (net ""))
 (segment (start 183.17 97.53) (end 183.17 96.39) (width 0.2) (layer "F.Cu") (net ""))
 (segment (start 187.06 98.96) (end 185.74 97.64) (width 0.2) (layer "F.Cu") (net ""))
 (segment (start 180 79.5) (end 179 78.5) (width 0.2) (layer "F.Cu") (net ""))
 (segment (start 191.4 83.38) (end 189.03 81.01) (width 0.2) (layer "F.Cu") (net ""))
 (segment (start 146.42 92.08) (end 146.42 101) (width 0.2) (layer "F.Cu") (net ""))
 (segment (start 178.5 94.5) (end 180 93) (width 0.2) (layer "F.Cu") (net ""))
 (segment (start 156.58 101) (end 156.58 95.61) (width 0.2) (layer "F.Cu") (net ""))
 (segment (start 164.1 90.2) (end 148.3 90.2) (width 0.2) (layer "F.Cu") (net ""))
 (segment (start 187.39 107.01) (end 191.4 103) (width 0.2) (layer "F.Cu") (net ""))
 (segment (start 193.6 94.09) (end 193.6 93.59) (width 0.2) (layer "F.Cu") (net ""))
 (segment (start 197.5 114) (end 197.25 113.75) (width 0.2) (layer "F.Cu") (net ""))
 (segment (start 164.2 101) (end 164.2 102.65) (width 0.2) (layer "F.Cu") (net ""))
 (segment (start 199 103) (end 199 111) (width 0.2) (layer "F.Cu") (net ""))
 (segment (start 183.28 97.64) (end 183.17 97.53) (width 0.2) (layer "F.Cu") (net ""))
 (segment (start 186 115) (end 184.52 116.48) (width 0.2) (layer "F.Cu") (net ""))
 (segment (start 184.52 116.48) (end 184.52 118.78) (width 0.2) (layer "F.Cu") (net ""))
 (segment (start 204.1 87.59) (end 204.5 87.99) (width 0.2) (layer "F.Cu") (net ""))
 (segment (start 204.5 87.99) (end 204.5 90.9) (width 0.2) (layer "F.Cu") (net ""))
 (segment (start 168.56 107.01) (end 187.39 107.01) (width 0.2) (layer "F.Cu") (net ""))
 (segment (start 179 78.5) (end 172.5 78.5) (width 0.2) (layer "F.Cu") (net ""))
 (segment (start 203 114) (end 197.5 114) (width 0.2) (layer "F.Cu") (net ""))
 (segment (start 179.1 112.09) (end 182.1 109.09) (width 0.2) (layer "F.Cu") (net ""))
 (segment (start 182.26 86.59) (end 182.26 85.36) (width 0.2) (layer "F.Cu") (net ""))
 (segment (start 178.74 77.62) (end 179.29 77.07) (width 0.2) (layer "F.Cu") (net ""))
 (segment (start 164.1 105.59) (end 167.1 108.59) (width 0.2) (layer "F.Cu") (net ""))
 (segment (start 181.16 75.2) (end 185.79 75.2) (width 0.2) (layer "F.Cu") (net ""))
 (segment (start 185.79 75.2) (end 189.03 78.44) (width 0.2) (layer "F.Cu") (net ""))
 (segment (start 180.6 86.09) (end 181.1 86.59) (width 0.2) (layer "F.Cu") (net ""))
 (segment (start 180 93) (end 180 79.5) (width 0.2) (layer "F.Cu") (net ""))
 (segment (start 185.74 97.64) (end 183.28 97.64) (width 0.2) (layer "F.Cu") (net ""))
 (segment (start 181 95.5) (end 182.26 94.24) (width 0.2) (layer "F.Cu") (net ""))
 (segment (start 204.16 118) (end 204.16 115.16) (width 0.2) (layer "F.Cu") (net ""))
 (segment (start 195.6 102.09) (end 196.6 102.09) (width 0.2) (layer "F.Cu") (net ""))
 (segment (start 195.1 96.09) (end 195.6 95.59) (width 0.2) (layer "F.Cu") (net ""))
 (segment (start 159.12 101) (end 159.12 97.38) (width 0.2) (layer "F.Cu") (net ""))
 (segment (start 159.6 114.09) (end 194.1 114.09) (width 0.2) (layer "F.Cu") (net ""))
 (segment (start 194.6 95.09) (end 193.6 94.09) (width 0.2) (layer "F.Cu") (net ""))
 (segment (start 197.25 101.25) (end 199 103) (width 0.2) (layer "F.Cu") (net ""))
 (segment (start 185.04 93.7) (end 185.77 92.97) (width 0.2) (layer "F.Cu") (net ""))
 (segment (start 161 95.5) (end 181 95.5) (width 0.2) (layer "F.Cu") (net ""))
 (segment (start 196 115) (end 195.5 115) (width 0.2) (layer "F.Cu") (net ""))
 (segment (start 199.5 111.5) (end 204.5 111.5) (width 0.2) (layer "F.Cu") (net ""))
 (segment (start 157.1 95.09) (end 180.1 95.09) (width 0.2) (layer "F.Cu") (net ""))
 (segment (start 182.26 79.3) (end 180.03 77.07) (width 0.2) (layer "F.Cu") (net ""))
 (segment (start 195.1 113.09) (end 195.1 102.59) (width 0.2) (layer "F.Cu") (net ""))
 (segment (start 151.5 105.99) (end 159.6 114.09) (width 0.2) (layer "F.Cu") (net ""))
 (segment (start 185.77 92.97) (end 185.77 91.5) (width 0.2) (layer "F.Cu") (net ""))
 (segment (start 199 111) (end 199.5 111.5) (width 0.2) (layer "F.Cu") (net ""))
 (segment (start 172.5 78.5) (end 172 78) (width 0.2) (layer "F.Cu") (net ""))
 (segment (start 179.29 77.07) (end 181.16 75.2) (width 0.2) (layer "F.Cu") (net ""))
 (segment (start 159.12 97.38) (end 161 95.5) (width 0.2) (layer "F.Cu") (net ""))
 (segment (start 151.5 101) (end 151.5 105.99) (width 0.2) (layer "F.Cu") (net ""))
 (via (at 178.1 108.59) (size 0.6) (drill 0.3) (layers "F.Cu" "B.Cu") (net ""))
 (via (at 182.1 109.09) (size 0.6) (drill 0.3) (layers "F.Cu" "B.Cu") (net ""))
 (via (at 185.6 104.59) (size 0.6) (drill 0.3) (layers "F.Cu" "B.Cu") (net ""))
 (via (at 169.6 112.09) (size 0.6) (drill 0.3) (layers "F.Cu" "B.Cu") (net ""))
 (via (at 192.1 102.59) (size 0.6) (drill 0.3) (layers "F.Cu" "B.Cu") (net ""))
 (via (at 194.6 95.09) (size 0.6) (drill 0.3) (layers "F.Cu" "B.Cu") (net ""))
 (via (at 180.6 82.09) (size 0.6) (drill 0.3) (layers "F.Cu" "B.Cu") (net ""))
 (via (at 193.5 97.5) (size 0.6) (drill 0.3) (layers "F.Cu" "B.Cu") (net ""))
 (via (at 144.76 95.07) (size 0.6) (drill 0.3) (layers "F.Cu" "B.Cu") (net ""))
 (via (at 196.6 102.09) (size 0.6) (drill 0.3) (layers "F.Cu" "B.Cu") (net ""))
 (via (at 181.6 87.59) (size 0.6) (drill 0.3) (layers "F.Cu" "B.Cu") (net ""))
 (via (at 196 115) (size 0.6) (drill 0.3) (layers "F.Cu" "B.Cu") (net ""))
 (via (at 183.1 115.09) (size 0.6) (drill 0.3) (layers "F.Cu" "B.Cu") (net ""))
 (via (at 195.1 96.59) (size 0.6) (drill 0.3) (layers "F.Cu" "B.Cu") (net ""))
 (via (at 178.1 108.59) (size 0.6) (drill 0.3) (layers "F.Cu" "B.Cu") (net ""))
 (via (at 162.1 105.59) (size 0.6) (drill 0.3) (layers "F.Cu" "B.Cu") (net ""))
 (segment (start 184.5 91.5) (end 184.5 90.5) (width 0.2) (layer "B.Cu") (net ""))
 (segment (start 169.67 95.07) (end 170.15 94.59) (width 0.2) (layer "B.Cu") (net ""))
 (segment (start 180.6 108.59) (end 186.6 102.59) (width 0.2) (layer "B.Cu") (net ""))
 (segment (start 191.76 78.84) (end 186.49 73.57) (width 0.2) (layer "B.Cu") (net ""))
 (segment (start 192.6 104.09) (end 195.6 101.09) (width 0.2) (layer "B.Cu") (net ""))
 (segment (start 170.15 89.8) (end 171.73 88.22) (width 0.2) (layer "B.Cu") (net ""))
 (segment (start 192.1 103.59) (end 186.6 103.59) (width 0.2) (layer "B.Cu") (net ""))
 (segment (start 195.1 99.59) (end 193.1 101.59) (width 0.2) (layer "B.Cu") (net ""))
 (segment (start 171.73 88.22) (end 189.88 88.22) (width 0.2) (layer "B.Cu") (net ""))
 (segment (start 189.33 116.25) (end 191.08 118) (width 0.2) (layer "B.Cu") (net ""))
 (segment (start 184.5 90.5) (end 185.5 89.5) (width 0.2) (layer "B.Cu") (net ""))
 (segment (start 194.07 84.03) (end 194.07 81.38) (width 0.2) (layer "B.Cu") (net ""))
 (segment (start 193.1 102.59) (end 192.1 103.59) (width 0.2) (layer "B.Cu") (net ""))
 (segment (start 194.5 116) (end 201.5 116) (width 0.2) (layer "B.Cu") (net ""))
 (segment (start 194.07 78.84) (end 191.76 78.84) (width 0.2) (layer "B.Cu") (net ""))
 (segment (start 189.88 88.22) (end 194.07 84.03) (width 0.2) (layer "B.Cu") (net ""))
 (segment (start 143.88 101) (end 143.88 103.38) (width 0.2) (layer "B.Cu") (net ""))
 (segment (start 195.6 95.59) (end 195.1 95.09) (width 0.2) (layer "B.Cu") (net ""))
 (segment (start 179.6 81.09) (end 176.6 81.09) (width 0.2) (layer "B.Cu") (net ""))
 (segment (start 157.1 105.59) (end 162.1 105.59) (width 0.2) (layer "B.Cu") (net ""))
 (segment (start 154.04 118.78) (end 155.1 117.72) (width 0.2) (layer "B.Cu") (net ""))
 (segment (start 155.1 107.59) (end 157.1 105.59) (width 0.2) (layer "B.Cu") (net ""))
 (segment (start 191 97.5) (end 193.5 97.5) (width 0.2) (layer "B.Cu") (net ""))
 (segment (start 204.1 104.59) (end 204.5 104.19) (width 0.2) (layer "B.Cu") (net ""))
 (segment (start 181.6 86.59) (end 180.6 85.59) (width 0.2) (layer "B.Cu") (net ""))
 (segment (start 178.1 108.59) (end 180.6 108.59) (width 0.2) (layer "B.Cu") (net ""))
 (segment (start 196 95) (end 196 115) (width 0.2) (layer "B.Cu") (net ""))
 (segment (start 199.1 104.59) (end 204.1 104.59) (width 0.2) (layer "B.Cu") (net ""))
 (segment (start 195.6 101.09) (end 195.6 95.59) (width 0.2) (layer "B.Cu") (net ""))
 (segment (start 166.23 73.57) (end 164.1 75.7) (width 0.2) (layer "B.Cu") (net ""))
 (segment (start 180.6 82.09) (end 179.6 81.09) (width 0.2) (layer "B.Cu") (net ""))
 (segment (start 202.2 107.8) (end 204.5 107.8) (width 0.2) (layer "B.Cu") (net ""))
 (segment (start 182.1 109.09) (end 187.1 104.09) (width 0.2) (layer "B.Cu") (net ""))
 (segment (start 191.08 118) (end 194 118) (width 0.2) (layer "B.Cu") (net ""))
 (segment (start 143.88 103.38) (end 145 104.5) (width 0.2) (layer "B.Cu") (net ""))
 (segment (start 158.1 112.09) (end 169.6 112.09) (width 0.2) (layer "B.Cu") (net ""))
 (segment (start 194 116.5) (end 194.5 116) (width 0.2) (layer "B.Cu") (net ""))
 (segment (start 190.5 89.5) (end 196 95) (width 0.2) (layer "B.Cu") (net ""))
 (segment (start 195.1 96.59) (end 195.1 99.59) (width 0.2) (layer "B.Cu") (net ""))
 (segment (start 175.89 116.25) (end 189.33 116.25) (width 0.2) (layer "B.Cu") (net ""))
 (segment (start 196.6 102.09) (end 199.1 104.59) (width 0.2) (layer "B.Cu") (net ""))
 (segment (start 195.1 95.09) (end 194.6 95.09) (width 0.2) (layer "B.Cu") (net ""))
 (segment (start 164.14 104.5) (end 175.89 116.25) (width 0.2) (layer "B.Cu") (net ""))
 (segment (start 193.1 101.59) (end 193.1 102.59) (width 0.2) (layer "B.Cu") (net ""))
 (segment (start 187.04 93.54) (end 191 97.5) (width 0.2) (layer "B.Cu") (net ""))
 (segment (start 194 118) (end 194 116.5) (width 0.2) (layer "B.Cu") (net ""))
 (segment (start 204.5 104.19) (end 204.5 102) (width 0.2) (layer "B.Cu") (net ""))
 (segment (start 156.58 113.61) (end 158.1 112.09) (width 0.2) (layer "B.Cu") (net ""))
 (segment (start 186.49 73.57) (end 166.23 73.57) (width 0.2) (layer "B.Cu") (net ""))
 (segment (start 187.04 91.5) (end 187.04 93.54) (width 0.2) (layer "B.Cu") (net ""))
 (segment (start 186.6 103.59) (end 185.6 104.59) (width 0.2) (layer "B.Cu") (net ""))
 (segment (start 185.5 89.5) (end 190.5 89.5) (width 0.2) (layer "B.Cu") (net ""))
 (segment (start 156.58 118.78) (end 156.58 113.61) (width 0.2) (layer "B.Cu") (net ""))
 (segment (start 187.1 104.09) (end 192.6 104.09) (width 0.2) (layer "B.Cu") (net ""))
 (segment (start 155.1 117.72) (end 155.1 107.59) (width 0.2) (layer "B.Cu") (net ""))
 (segment (start 144.76 95.07) (end 169.67 95.07) (width 0.2) (layer "B.Cu") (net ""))
 (segment (start 201.5 108.5) (end 202.2 107.8) (width 0.2) (layer "B.Cu") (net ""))
 (segment (start 181.6 87.59) (end 181.6 86.59) (width 0.2) (layer "B.Cu") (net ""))
 (segment (start 170.15 94.59) (end 170.15 89.8) (width 0.2) (layer "B.Cu") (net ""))
 (segment (start 145 104.5) (end 164.14 104.5) (width 0.2) (layer "B.Cu") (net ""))
 (segment (start 186.6 102.59) (end 192.1 102.59) (width 0.2) (layer "B.Cu") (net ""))
 (segment (start 180.6 85.59) (end 176.6 85.59) (width 0.2) (layer "B.Cu") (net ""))
 (segment (start 201.5 116) (end 201.5 108.5) (width 0.2) (layer "B.Cu") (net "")))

